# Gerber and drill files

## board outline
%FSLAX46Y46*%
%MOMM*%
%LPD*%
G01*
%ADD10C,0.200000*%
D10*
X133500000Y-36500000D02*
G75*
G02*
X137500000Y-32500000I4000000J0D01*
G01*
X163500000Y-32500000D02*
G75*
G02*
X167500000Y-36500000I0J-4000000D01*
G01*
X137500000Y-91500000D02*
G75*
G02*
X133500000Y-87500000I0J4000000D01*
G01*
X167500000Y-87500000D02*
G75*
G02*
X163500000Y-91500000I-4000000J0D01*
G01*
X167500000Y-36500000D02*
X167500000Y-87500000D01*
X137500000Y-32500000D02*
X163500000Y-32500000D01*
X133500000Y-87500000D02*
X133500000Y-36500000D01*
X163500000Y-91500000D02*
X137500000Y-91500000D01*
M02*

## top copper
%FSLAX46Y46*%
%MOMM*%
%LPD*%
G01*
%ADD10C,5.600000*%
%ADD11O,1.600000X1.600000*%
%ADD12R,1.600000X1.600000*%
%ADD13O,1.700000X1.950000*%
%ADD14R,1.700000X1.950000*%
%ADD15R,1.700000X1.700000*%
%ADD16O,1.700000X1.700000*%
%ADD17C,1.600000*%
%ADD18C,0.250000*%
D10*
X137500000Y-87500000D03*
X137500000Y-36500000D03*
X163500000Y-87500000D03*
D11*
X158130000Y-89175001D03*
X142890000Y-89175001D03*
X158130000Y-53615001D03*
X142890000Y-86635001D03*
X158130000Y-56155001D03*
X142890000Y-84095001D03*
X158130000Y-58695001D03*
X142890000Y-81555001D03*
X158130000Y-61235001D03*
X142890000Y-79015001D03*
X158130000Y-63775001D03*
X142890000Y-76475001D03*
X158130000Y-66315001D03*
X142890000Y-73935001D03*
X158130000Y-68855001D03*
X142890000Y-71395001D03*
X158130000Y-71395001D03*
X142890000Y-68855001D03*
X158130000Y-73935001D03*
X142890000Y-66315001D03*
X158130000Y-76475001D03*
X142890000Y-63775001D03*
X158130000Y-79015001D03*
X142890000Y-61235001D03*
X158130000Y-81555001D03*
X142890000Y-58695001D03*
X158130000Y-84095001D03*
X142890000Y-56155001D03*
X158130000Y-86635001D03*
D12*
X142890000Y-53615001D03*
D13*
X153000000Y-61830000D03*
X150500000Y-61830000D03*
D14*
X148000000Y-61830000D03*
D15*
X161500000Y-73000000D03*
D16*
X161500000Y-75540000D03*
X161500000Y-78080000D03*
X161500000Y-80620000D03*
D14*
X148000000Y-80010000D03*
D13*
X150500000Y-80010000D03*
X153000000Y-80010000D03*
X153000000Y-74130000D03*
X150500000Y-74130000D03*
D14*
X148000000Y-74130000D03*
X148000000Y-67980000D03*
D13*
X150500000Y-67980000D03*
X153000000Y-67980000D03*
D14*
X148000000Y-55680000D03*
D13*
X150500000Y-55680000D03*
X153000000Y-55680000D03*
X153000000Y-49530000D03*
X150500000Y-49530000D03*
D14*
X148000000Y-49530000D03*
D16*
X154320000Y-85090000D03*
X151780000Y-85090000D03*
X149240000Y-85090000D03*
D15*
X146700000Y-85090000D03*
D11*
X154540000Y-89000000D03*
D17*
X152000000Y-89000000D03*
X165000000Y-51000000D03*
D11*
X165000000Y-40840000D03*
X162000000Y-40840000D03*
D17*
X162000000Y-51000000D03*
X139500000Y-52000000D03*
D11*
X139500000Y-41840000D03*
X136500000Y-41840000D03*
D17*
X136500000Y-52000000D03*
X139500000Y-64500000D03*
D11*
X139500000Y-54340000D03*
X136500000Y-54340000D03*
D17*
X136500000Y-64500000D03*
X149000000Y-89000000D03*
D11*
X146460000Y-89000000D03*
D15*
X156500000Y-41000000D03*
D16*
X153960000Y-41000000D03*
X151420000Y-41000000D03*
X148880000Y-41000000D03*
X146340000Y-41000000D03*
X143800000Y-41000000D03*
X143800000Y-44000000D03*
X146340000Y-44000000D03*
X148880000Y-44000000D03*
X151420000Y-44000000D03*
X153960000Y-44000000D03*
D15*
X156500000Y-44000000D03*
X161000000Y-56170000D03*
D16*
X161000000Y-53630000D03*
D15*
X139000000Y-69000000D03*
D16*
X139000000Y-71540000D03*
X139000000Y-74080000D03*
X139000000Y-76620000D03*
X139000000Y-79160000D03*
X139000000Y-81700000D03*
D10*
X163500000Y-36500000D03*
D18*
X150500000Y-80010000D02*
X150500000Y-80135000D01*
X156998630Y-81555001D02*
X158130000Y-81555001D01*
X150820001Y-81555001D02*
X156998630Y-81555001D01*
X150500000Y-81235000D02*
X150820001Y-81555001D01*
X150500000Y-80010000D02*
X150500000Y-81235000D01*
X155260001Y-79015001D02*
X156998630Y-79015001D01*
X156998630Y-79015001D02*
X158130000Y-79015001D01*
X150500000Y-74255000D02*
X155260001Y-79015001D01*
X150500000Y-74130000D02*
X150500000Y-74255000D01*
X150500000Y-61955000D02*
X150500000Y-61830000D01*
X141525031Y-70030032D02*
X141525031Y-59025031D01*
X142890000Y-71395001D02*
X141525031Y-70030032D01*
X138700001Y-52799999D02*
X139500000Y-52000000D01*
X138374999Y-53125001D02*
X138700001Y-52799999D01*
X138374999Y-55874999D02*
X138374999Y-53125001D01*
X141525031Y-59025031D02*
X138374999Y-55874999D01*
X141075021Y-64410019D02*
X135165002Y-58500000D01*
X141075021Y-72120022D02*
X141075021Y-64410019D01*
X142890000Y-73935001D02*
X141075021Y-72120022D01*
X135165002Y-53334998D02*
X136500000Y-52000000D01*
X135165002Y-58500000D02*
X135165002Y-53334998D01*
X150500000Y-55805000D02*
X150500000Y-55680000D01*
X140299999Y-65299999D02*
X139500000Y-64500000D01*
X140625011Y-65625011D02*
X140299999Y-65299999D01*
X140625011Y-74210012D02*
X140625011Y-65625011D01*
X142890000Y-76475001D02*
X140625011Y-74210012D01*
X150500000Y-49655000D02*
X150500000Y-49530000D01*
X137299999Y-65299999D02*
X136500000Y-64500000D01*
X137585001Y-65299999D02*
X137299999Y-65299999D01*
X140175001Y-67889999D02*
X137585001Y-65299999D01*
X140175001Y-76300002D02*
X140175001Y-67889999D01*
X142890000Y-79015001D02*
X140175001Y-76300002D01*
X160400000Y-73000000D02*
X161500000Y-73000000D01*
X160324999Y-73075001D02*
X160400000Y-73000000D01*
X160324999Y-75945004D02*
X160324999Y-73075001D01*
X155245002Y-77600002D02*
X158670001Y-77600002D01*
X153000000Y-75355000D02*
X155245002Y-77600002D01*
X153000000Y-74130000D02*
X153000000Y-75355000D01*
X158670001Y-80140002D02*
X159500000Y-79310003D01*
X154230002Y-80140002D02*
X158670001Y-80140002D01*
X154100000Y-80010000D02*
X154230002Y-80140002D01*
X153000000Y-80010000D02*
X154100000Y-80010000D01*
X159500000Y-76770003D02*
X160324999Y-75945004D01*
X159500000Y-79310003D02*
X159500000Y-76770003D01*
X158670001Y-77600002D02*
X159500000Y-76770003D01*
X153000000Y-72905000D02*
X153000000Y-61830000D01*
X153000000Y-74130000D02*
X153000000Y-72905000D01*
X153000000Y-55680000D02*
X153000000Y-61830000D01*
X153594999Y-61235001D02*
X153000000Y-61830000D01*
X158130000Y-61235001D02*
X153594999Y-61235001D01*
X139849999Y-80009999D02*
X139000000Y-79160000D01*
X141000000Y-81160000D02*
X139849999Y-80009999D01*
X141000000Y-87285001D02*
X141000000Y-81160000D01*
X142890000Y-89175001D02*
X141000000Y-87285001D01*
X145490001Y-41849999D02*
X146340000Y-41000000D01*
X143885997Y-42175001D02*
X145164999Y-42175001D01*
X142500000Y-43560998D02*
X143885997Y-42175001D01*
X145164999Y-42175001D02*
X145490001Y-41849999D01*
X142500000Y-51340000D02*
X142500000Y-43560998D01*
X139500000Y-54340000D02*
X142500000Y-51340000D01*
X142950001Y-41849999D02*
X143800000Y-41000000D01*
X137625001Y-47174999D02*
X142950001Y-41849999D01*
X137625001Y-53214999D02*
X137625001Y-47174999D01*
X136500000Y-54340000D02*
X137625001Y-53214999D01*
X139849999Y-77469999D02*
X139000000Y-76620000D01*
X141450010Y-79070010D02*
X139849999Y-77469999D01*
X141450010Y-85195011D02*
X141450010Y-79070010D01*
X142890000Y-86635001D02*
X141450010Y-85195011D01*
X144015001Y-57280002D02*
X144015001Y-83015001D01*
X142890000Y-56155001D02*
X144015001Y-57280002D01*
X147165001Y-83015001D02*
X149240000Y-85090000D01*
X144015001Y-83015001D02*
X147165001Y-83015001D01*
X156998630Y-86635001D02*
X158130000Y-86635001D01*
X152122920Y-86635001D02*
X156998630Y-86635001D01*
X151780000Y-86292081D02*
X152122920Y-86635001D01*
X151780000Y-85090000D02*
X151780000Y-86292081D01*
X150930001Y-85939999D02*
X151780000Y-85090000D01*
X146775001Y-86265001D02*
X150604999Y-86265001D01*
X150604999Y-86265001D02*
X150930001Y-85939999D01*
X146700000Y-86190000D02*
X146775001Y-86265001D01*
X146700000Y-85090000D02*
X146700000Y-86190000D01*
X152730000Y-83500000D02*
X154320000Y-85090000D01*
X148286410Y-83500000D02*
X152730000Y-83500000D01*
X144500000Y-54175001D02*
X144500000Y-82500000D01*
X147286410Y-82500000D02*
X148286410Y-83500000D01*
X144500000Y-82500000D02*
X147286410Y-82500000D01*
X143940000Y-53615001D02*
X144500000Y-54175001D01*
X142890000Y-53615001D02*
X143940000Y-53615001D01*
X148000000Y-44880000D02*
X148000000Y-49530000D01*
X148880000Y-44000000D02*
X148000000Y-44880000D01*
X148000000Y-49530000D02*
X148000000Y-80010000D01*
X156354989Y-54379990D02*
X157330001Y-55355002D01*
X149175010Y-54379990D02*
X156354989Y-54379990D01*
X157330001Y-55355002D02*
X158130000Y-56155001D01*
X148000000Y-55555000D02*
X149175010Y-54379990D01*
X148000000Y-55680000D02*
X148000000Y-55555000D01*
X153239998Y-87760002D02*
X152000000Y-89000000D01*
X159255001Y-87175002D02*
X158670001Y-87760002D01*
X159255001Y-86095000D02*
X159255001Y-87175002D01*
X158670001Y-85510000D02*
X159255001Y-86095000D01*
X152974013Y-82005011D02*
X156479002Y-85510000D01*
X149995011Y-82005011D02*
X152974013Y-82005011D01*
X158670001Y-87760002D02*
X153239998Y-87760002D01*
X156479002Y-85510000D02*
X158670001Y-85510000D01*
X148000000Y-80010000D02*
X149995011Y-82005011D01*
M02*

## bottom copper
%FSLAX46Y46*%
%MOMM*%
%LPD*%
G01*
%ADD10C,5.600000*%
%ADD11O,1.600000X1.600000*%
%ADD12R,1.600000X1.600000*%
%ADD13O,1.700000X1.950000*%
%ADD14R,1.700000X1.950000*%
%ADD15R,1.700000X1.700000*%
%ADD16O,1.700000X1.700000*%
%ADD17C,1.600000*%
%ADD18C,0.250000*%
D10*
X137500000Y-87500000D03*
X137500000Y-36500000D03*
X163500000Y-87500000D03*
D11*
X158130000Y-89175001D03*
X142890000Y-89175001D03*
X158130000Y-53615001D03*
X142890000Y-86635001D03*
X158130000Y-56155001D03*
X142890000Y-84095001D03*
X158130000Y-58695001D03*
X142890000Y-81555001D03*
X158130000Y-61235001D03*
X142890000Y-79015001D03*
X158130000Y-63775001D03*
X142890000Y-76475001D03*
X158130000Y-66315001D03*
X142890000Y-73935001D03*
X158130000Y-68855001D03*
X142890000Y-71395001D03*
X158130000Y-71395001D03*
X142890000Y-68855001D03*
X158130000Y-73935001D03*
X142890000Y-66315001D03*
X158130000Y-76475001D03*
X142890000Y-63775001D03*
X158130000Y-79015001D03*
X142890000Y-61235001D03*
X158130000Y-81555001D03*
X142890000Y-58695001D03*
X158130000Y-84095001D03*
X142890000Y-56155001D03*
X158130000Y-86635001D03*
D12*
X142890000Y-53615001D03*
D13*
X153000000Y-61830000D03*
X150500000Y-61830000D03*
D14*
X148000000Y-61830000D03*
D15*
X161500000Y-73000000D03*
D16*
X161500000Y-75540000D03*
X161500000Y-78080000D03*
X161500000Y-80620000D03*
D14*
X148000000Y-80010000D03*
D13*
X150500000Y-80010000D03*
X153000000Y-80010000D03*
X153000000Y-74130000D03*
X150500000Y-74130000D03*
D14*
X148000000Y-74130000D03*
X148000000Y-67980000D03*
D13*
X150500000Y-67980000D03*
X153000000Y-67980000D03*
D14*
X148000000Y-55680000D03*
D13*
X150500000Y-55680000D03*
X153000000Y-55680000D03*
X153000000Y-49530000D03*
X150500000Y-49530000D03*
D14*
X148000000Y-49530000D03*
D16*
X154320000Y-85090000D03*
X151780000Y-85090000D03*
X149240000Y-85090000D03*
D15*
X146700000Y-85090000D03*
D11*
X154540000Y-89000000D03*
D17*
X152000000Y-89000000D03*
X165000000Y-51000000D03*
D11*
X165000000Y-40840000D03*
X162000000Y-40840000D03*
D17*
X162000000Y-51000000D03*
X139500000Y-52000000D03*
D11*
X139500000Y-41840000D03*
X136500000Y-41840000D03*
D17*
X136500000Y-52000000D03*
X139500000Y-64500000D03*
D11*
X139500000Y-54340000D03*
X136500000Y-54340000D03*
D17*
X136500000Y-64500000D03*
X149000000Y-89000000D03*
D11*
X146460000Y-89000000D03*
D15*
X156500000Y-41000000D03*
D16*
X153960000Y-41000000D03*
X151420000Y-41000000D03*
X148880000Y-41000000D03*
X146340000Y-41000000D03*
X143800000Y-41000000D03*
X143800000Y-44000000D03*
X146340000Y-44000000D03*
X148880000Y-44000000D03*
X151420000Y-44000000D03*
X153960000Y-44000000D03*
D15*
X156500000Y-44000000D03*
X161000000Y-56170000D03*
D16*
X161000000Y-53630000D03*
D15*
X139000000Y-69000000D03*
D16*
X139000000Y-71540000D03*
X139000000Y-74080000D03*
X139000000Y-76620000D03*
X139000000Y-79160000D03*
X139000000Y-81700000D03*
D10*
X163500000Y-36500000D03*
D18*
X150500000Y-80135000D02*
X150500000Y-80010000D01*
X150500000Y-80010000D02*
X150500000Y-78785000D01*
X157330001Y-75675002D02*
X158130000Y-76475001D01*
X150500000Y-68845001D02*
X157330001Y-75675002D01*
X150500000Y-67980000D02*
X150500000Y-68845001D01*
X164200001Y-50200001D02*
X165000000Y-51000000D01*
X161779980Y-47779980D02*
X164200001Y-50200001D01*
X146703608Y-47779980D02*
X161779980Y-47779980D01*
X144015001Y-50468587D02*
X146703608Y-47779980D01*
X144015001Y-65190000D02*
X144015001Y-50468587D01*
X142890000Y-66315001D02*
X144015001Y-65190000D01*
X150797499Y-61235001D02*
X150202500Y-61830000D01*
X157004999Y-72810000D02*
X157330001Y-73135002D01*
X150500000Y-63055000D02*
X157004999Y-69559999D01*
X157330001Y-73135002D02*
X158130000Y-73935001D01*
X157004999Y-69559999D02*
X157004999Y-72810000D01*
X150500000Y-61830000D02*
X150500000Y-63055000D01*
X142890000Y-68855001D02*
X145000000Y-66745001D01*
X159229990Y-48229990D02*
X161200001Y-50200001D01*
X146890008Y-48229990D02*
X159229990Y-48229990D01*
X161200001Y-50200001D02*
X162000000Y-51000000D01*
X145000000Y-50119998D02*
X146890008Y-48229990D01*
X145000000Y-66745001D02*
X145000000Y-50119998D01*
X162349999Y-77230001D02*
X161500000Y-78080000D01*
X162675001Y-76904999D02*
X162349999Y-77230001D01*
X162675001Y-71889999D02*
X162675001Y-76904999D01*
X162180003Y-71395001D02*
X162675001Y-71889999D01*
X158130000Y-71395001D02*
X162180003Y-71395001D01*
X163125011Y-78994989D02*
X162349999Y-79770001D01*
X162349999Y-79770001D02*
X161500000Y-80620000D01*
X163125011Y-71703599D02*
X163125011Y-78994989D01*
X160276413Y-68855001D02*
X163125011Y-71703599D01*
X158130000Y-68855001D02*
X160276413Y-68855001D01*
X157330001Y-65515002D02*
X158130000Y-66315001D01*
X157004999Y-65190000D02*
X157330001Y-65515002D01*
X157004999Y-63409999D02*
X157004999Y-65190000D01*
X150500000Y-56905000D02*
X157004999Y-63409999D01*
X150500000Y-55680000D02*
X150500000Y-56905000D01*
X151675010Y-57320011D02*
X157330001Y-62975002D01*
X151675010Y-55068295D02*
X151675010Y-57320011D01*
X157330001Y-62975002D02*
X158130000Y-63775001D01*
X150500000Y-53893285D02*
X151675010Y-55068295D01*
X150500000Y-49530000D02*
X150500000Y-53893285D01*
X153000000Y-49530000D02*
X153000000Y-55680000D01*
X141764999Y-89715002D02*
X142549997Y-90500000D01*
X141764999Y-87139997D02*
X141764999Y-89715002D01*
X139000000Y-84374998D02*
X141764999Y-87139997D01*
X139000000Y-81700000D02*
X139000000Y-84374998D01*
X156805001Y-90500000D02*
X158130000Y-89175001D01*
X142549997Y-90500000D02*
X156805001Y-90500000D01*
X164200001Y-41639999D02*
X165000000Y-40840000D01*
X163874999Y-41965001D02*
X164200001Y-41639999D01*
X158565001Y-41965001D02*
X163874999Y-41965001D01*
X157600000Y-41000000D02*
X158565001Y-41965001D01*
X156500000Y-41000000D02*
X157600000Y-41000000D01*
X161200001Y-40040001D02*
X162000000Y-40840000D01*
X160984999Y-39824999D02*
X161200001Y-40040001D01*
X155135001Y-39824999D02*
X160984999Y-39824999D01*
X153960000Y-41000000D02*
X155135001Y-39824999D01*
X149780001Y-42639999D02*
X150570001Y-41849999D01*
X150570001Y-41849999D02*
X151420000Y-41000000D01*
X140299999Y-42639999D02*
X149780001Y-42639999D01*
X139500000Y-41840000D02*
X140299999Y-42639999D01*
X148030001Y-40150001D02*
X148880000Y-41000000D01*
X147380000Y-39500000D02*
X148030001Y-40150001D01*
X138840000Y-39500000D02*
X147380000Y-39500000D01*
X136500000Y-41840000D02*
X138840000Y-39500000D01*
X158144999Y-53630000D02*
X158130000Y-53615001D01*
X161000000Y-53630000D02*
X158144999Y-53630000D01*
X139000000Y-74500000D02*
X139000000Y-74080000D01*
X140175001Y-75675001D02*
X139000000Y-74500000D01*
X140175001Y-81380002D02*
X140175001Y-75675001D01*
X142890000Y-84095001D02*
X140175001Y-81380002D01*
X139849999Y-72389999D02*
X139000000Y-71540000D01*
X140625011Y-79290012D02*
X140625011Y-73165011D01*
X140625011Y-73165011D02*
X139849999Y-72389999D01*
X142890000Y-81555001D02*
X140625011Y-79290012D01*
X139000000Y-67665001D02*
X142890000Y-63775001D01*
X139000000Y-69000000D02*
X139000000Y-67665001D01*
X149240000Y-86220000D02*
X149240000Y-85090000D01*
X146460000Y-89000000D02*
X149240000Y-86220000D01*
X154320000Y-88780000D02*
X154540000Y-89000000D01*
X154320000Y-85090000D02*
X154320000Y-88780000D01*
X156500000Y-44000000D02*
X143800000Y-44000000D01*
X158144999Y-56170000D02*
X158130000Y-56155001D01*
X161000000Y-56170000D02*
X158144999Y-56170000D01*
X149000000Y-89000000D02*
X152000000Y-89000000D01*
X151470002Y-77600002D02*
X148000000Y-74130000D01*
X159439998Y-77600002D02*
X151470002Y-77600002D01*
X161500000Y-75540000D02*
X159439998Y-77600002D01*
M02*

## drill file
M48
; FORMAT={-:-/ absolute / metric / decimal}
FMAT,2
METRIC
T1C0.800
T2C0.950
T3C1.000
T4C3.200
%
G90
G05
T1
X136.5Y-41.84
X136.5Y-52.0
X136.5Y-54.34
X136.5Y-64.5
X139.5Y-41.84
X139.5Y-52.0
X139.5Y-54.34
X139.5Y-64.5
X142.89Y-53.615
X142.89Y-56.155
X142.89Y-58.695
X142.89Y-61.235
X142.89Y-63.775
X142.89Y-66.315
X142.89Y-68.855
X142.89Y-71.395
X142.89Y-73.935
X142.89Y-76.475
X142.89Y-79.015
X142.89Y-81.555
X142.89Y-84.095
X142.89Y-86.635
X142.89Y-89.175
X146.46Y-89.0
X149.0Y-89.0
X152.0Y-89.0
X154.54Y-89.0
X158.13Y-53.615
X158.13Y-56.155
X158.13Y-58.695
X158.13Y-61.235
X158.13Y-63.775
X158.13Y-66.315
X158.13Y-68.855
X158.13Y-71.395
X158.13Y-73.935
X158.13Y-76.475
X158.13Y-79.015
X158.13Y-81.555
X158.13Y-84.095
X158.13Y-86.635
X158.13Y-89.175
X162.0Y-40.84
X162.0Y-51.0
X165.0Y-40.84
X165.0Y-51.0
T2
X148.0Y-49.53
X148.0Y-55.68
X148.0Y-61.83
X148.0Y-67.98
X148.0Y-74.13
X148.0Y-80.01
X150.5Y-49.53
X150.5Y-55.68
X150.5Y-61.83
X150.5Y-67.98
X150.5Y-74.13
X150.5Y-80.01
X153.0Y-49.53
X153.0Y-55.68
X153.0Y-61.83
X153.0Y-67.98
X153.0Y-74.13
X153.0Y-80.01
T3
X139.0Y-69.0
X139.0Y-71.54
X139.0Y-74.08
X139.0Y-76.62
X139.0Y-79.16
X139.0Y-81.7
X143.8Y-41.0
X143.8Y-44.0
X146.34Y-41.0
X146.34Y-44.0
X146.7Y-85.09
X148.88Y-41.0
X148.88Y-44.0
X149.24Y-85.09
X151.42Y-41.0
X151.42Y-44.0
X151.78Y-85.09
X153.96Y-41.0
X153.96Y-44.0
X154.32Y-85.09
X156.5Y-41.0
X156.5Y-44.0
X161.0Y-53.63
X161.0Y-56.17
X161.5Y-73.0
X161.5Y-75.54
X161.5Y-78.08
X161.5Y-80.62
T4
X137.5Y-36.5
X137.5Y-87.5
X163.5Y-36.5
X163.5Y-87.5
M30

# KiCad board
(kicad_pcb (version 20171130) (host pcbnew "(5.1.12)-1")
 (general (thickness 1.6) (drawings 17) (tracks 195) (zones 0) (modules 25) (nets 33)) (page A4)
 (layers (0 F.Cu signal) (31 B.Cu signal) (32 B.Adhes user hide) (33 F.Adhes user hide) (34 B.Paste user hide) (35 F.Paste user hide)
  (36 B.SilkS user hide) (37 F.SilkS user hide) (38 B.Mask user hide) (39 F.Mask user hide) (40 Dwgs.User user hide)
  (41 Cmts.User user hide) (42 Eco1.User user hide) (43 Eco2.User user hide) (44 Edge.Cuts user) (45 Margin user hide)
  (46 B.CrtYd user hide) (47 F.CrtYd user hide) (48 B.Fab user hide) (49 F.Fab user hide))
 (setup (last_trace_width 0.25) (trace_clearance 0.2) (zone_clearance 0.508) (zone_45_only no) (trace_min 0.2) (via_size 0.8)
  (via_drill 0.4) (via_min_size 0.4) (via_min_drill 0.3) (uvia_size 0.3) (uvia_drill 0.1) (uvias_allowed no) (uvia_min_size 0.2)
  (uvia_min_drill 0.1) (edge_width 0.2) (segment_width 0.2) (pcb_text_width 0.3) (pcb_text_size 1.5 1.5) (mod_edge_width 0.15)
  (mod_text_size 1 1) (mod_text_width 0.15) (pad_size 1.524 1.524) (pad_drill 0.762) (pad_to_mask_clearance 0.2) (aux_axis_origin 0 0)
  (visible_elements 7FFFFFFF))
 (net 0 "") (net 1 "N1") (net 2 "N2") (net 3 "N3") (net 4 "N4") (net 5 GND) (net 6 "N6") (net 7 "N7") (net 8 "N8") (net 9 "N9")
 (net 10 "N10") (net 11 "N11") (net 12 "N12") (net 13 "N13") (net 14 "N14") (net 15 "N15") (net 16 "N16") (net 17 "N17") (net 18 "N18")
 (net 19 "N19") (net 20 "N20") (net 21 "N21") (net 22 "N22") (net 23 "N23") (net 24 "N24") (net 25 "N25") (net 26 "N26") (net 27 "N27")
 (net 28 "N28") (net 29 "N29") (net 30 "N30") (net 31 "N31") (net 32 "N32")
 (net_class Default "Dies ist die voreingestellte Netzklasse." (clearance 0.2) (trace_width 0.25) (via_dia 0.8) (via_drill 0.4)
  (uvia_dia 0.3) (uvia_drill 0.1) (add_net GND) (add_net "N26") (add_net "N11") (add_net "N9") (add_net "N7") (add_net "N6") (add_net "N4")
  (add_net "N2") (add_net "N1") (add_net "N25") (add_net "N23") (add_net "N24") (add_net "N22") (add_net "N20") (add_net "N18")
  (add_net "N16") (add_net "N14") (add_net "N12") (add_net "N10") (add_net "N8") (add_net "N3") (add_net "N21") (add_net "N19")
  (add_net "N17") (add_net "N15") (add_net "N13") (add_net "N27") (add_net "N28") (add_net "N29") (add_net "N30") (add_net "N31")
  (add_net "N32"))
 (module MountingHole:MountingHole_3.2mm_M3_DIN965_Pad (layer F.Cu) (at 137.5 87.5)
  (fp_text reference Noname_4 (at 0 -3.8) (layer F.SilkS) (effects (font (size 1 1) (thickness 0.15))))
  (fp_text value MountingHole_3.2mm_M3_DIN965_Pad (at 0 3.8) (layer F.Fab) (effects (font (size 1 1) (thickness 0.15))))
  (pad 1 thru_hole circle (at 0 0) (size 5.6 5.6) (drill 3.2) (layers *.Cu *.Mask)))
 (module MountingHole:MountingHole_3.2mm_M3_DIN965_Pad (layer F.Cu) (at 137.5 36.5)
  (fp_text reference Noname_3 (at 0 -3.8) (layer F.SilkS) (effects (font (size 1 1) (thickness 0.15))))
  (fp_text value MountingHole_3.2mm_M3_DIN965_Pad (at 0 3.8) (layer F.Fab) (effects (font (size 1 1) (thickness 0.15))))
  (pad 1 thru_hole circle (at 0 0) (size 5.6 5.6) (drill 3.2) (layers *.Cu *.Mask)))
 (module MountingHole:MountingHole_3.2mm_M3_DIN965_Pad (layer F.Cu) (at 163.5 87.5)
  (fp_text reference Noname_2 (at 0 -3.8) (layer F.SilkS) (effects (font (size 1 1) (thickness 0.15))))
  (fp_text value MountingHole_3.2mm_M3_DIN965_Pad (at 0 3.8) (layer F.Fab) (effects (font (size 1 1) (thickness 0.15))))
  (pad 1 thru_hole circle (at 0 0) (size 5.6 5.6) (drill 3.2) (layers *.Cu *.Mask)))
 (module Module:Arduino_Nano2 (layer F.Cu) (at 142.89 53.615001)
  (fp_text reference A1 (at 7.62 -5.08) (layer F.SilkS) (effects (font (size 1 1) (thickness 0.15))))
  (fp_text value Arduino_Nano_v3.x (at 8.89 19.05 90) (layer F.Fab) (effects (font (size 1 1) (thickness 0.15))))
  (pad 16 thru_hole oval (at 15.24 35.56) (size 1.6 1.6) (drill 0.8) (layers *.Cu *.Mask) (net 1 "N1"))
  (pad 15 thru_hole oval (at 0 35.56) (size 1.6 1.6) (drill 0.8) (layers *.Cu *.Mask) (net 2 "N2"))
  (pad 30 thru_hole oval (at 15.24 0) (size 1.6 1.6) (drill 0.8) (layers *.Cu *.Mask) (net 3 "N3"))
  (pad 14 thru_hole oval (at 0 33.02) (size 1.6 1.6) (drill 0.8) (layers *.Cu *.Mask) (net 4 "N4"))
  (pad 29 thru_hole oval (at 15.24 2.54) (size 1.6 1.6) (drill 0.8) (layers *.Cu *.Mask) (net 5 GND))
  (pad 13 thru_hole oval (at 0 30.48) (size 1.6 1.6) (drill 0.8) (layers *.Cu *.Mask) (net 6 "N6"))
  (pad 28 thru_hole oval (at 15.24 5.08) (size 1.6 1.6) (drill 0.8) (layers *.Cu *.Mask))
  (pad 12 thru_hole oval (at 0 27.94) (size 1.6 1.6) (drill 0.8) (layers *.Cu *.Mask) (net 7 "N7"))
  (pad 27 thru_hole oval (at 15.24 7.62) (size 1.6 1.6) (drill 0.8) (layers *.Cu *.Mask) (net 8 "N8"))
  (pad 11 thru_hole oval (at 0 25.4) (size 1.6 1.6) (drill 0.8) (layers *.Cu *.Mask) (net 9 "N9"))
  (pad 26 thru_hole oval (at 15.24 10.16) (size 1.6 1.6) (drill 0.8) (layers *.Cu *.Mask) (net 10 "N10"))
  (pad 10 thru_hole oval (at 0 22.86) (size 1.6 1.6) (drill 0.8) (layers *.Cu *.Mask) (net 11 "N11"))
  (pad 25 thru_hole oval (at 15.24 12.7) (size 1.6 1.6) (drill 0.8) (layers *.Cu *.Mask) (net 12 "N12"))
  (pad 9 thru_hole oval (at 0 20.32) (size 1.6 1.6) (drill 0.8) (layers *.Cu *.Mask) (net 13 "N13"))
  (pad 24 thru_hole oval (at 15.24 15.24) (size 1.6 1.6) (drill 0.8) (layers *.Cu *.Mask) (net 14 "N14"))
  (pad 8 thru_hole oval (at 0 17.78) (size 1.6 1.6) (drill 0.8) (layers *.Cu *.Mask) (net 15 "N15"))
  (pad 23 thru_hole oval (at 15.24 17.78) (size 1.6 1.6) (drill 0.8) (layers *.Cu *.Mask) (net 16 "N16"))
  (pad 7 thru_hole oval (at 0 15.24) (size 1.6 1.6) (drill 0.8) (layers *.Cu *.Mask) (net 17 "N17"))
  (pad 22 thru_hole oval (at 15.24 20.32) (size 1.6 1.6) (drill 0.8) (layers *.Cu *.Mask) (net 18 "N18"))
  (pad 6 thru_hole oval (at 0 12.7) (size 1.6 1.6) (drill 0.8) (layers *.Cu *.Mask) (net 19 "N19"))
  (pad 21 thru_hole oval (at 15.24 22.86) (size 1.6 1.6) (drill 0.8) (layers *.Cu *.Mask) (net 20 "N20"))
  (pad 5 thru_hole oval (at 0 10.16) (size 1.6 1.6) (drill 0.8) (layers *.Cu *.Mask) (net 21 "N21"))
  (pad 20 thru_hole oval (at 15.24 25.4) (size 1.6 1.6) (drill 0.8) (layers *.Cu *.Mask) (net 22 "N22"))
  (pad 4 thru_hole oval (at 0 7.62) (size 1.6 1.6) (drill 0.8) (layers *.Cu *.Mask))
  (pad 19 thru_hole oval (at 15.24 27.94) (size 1.6 1.6) (drill 0.8) (layers *.Cu *.Mask) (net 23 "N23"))
  (pad 3 thru_hole oval (at 0 5.08) (size 1.6 1.6) (drill 0.8) (layers *.Cu *.Mask))
  (pad 18 thru_hole oval (at 15.24 30.48) (size 1.6 1.6) (drill 0.8) (layers *.Cu *.Mask))
  (pad 2 thru_hole oval (at 0 2.54) (size 1.6 1.6) (drill 0.8) (layers *.Cu *.Mask) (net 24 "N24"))
  (pad 17 thru_hole oval (at 15.24 33.02) (size 1.6 1.6) (drill 0.8) (layers *.Cu *.Mask) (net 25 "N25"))
  (pad 1 thru_hole rect (at 0 0) (size 1.6 1.6) (drill 0.8) (layers *.Cu *.Mask) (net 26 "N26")))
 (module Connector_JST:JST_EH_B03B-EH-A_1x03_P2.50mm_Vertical (layer F.Cu) (at 148 61.83)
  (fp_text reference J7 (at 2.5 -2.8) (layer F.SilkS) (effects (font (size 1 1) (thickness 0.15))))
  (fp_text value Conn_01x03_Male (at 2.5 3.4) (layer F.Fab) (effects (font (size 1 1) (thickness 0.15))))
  (pad 3 thru_hole oval (at 5 0) (size 1.7 1.95) (drill 0.95) (layers *.Cu *.Mask) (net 8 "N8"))
  (pad 2 thru_hole oval (at 2.5 0) (size 1.7 1.95) (drill 0.95) (layers *.Cu *.Mask) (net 18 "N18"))
  (pad 1 thru_hole rect (at 0 0) (size 1.7 1.95) (drill 0.95) (layers *.Cu *.Mask) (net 5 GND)))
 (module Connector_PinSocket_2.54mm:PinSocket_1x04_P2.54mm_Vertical (layer F.Cu) (at 161.5 73)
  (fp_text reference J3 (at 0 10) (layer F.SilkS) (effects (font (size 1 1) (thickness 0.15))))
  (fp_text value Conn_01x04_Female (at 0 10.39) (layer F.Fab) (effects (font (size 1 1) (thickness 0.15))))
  (pad 1 thru_hole rect (at 0 0) (size 1.7 1.7) (drill 1) (layers *.Cu *.Mask) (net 8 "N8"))
  (pad 2 thru_hole oval (at 0 2.54) (size 1.7 1.7) (drill 1) (layers *.Cu *.Mask) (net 5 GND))
  (pad 3 thru_hole oval (at 0 5.08) (size 1.7 1.7) (drill 1) (layers *.Cu *.Mask) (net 16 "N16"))
  (pad 4 thru_hole oval (at 0 7.62) (size 1.7 1.7) (drill 1) (layers *.Cu *.Mask) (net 14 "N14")))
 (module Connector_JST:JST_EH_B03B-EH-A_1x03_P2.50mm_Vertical (layer F.Cu) (at 148 80.01)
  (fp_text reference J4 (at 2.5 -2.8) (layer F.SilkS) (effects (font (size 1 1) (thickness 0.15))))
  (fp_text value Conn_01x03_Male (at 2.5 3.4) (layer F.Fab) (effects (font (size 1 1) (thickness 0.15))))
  (pad 1 thru_hole rect (at 0 0) (size 1.7 1.95) (drill 0.95) (layers *.Cu *.Mask) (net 5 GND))
  (pad 2 thru_hole oval (at 2.5 0) (size 1.7 1.95) (drill 0.95) (layers *.Cu *.Mask) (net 23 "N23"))
  (pad 3 thru_hole oval (at 5 0) (size 1.7 1.95) (drill 0.95) (layers *.Cu *.Mask) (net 8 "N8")))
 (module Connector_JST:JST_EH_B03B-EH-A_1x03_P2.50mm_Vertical (layer F.Cu) (at 148 74.13)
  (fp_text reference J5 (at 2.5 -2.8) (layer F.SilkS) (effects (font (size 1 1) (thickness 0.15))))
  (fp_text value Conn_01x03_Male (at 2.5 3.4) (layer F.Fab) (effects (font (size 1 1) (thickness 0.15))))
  (pad 3 thru_hole oval (at 5 0) (size 1.7 1.95) (drill 0.95) (layers *.Cu *.Mask) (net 8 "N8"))
  (pad 2 thru_hole oval (at 2.5 0) (size 1.7 1.95) (drill 0.95) (layers *.Cu *.Mask) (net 22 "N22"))
  (pad 1 thru_hole rect (at 0 0) (size 1.7 1.95) (drill 0.95) (layers *.Cu *.Mask) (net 5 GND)))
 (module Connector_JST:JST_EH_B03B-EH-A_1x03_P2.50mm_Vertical (layer F.Cu) (at 148 67.98)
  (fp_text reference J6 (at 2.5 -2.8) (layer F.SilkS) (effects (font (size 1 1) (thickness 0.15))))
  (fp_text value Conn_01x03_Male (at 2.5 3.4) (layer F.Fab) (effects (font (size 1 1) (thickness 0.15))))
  (pad 1 thru_hole rect (at 0 0) (size 1.7 1.95) (drill 0.95) (layers *.Cu *.Mask) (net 5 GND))
  (pad 2 thru_hole oval (at 2.5 0) (size 1.7 1.95) (drill 0.95) (layers *.Cu *.Mask) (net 20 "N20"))
  (pad 3 thru_hole oval (at 5 0) (size 1.7 1.95) (drill 0.95) (layers *.Cu *.Mask) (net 8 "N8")))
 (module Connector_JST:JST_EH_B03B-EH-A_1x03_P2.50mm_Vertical (layer F.Cu) (at 148 55.68)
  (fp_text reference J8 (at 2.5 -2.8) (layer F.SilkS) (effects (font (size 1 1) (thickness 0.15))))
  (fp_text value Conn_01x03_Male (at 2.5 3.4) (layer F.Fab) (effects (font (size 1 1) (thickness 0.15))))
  (pad 1 thru_hole rect (at 0 0) (size 1.7 1.95) (drill 0.95) (layers *.Cu *.Mask) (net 5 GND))
  (pad 2 thru_hole oval (at 2.5 0) (size 1.7 1.95) (drill 0.95) (layers *.Cu *.Mask) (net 12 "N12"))
  (pad 3 thru_hole oval (at 5 0) (size 1.7 1.95) (drill 0.95) (layers *.Cu *.Mask) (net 8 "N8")))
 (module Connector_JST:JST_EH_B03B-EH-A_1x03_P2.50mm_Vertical (layer F.Cu) (at 148 49.53)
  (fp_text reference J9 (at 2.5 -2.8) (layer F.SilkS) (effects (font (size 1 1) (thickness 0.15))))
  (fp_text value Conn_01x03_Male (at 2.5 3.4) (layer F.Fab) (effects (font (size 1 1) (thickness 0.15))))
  (pad 3 thru_hole oval (at 5 0) (size 1.7 1.95) (drill 0.95) (layers *.Cu *.Mask) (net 8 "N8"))
  (pad 2 thru_hole oval (at 2.5 0) (size 1.7 1.95) (drill 0.95) (layers *.Cu *.Mask) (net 10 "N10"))
  (pad 1 thru_hole rect (at 0 0) (size 1.7 1.95) (drill 0.95) (layers *.Cu *.Mask) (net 5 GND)))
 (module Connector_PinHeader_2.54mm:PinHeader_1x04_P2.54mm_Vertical (layer F.Cu) (at 146.7 85.09 90)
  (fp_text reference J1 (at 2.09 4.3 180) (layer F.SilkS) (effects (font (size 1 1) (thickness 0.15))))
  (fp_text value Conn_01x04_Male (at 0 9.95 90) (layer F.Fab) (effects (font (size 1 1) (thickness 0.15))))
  (pad 4 thru_hole oval (at 0 7.62 90) (size 1.7 1.7) (drill 1) (layers *.Cu *.Mask) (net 26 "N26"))
  (pad 3 thru_hole oval (at 0 5.08 90) (size 1.7 1.7) (drill 1) (layers *.Cu *.Mask) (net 25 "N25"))
  (pad 2 thru_hole oval (at 0 2.54 90) (size 1.7 1.7) (drill 1) (layers *.Cu *.Mask) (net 24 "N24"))
  (pad 1 thru_hole rect (at 0 0 90) (size 1.7 1.7) (drill 1) (layers *.Cu *.Mask) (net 25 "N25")))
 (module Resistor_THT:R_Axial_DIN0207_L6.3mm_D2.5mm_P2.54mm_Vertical (layer F.Cu) (at 152 89)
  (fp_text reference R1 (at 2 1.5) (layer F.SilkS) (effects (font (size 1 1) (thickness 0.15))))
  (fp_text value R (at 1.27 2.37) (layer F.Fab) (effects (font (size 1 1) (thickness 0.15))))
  (pad 2 thru_hole oval (at 2.54 0) (size 1.6 1.6) (drill 0.8) (layers *.Cu *.Mask) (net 26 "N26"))
  (pad 1 thru_hole circle (at 0 0) (size 1.6 1.6) (drill 0.8) (layers *.Cu *.Mask) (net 5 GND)))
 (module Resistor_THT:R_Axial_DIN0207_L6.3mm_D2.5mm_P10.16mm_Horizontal (layer F.Cu) (at 165 51 90)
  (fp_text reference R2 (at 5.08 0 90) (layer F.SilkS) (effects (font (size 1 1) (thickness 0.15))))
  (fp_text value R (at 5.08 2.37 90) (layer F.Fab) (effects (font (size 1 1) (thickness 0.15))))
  (pad 1 thru_hole circle (at 0 0 90) (size 1.6 1.6) (drill 0.8) (layers *.Cu *.Mask) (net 19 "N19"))
  (pad 2 thru_hole oval (at 10.16 0 90) (size 1.6 1.6) (drill 0.8) (layers *.Cu *.Mask) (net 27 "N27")))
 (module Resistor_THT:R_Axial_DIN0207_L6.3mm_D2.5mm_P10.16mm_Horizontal (layer F.Cu) (at 162 51 90)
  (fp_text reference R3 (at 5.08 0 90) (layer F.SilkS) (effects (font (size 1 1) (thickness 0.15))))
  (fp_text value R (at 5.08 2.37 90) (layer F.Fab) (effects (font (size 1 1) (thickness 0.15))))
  (pad 2 thru_hole oval (at 10.16 0 90) (size 1.6 1.6) (drill 0.8) (layers *.Cu *.Mask) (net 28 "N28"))
  (pad 1 thru_hole circle (at 0 0 90) (size 1.6 1.6) (drill 0.8) (layers *.Cu *.Mask) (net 17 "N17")))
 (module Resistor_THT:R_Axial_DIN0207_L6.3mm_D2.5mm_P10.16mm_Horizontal (layer F.Cu) (at 139.5 52 90)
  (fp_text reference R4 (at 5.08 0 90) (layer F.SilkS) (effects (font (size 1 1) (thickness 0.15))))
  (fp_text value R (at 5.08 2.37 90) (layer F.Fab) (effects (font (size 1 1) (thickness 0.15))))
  (pad 1 thru_hole circle (at 0 0 90) (size 1.6 1.6) (drill 0.8) (layers *.Cu *.Mask) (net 15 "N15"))
  (pad 2 thru_hole oval (at 10.16 0 90) (size 1.6 1.6) (drill 0.8) (layers *.Cu *.Mask) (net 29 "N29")))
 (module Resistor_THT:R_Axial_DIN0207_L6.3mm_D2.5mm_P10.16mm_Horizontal (layer F.Cu) (at 136.5 52 90)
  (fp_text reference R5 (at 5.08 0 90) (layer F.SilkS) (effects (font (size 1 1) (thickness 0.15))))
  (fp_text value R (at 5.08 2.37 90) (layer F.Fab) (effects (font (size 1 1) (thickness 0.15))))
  (pad 2 thru_hole oval (at 10.16 0 90) (size 1.6 1.6) (drill 0.8) (layers *.Cu *.Mask) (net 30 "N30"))
  (pad 1 thru_hole circle (at 0 0 90) (size 1.6 1.6) (drill 0.8) (layers *.Cu *.Mask) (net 13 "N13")))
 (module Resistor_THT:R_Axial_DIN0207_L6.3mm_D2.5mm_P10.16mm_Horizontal (layer F.Cu) (at 139.5 64.5 90)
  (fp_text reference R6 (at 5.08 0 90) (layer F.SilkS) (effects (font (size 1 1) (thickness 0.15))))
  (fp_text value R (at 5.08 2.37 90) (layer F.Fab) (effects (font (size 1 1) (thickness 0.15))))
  (pad 1 thru_hole circle (at 0 0 90) (size 1.6 1.6) (drill 0.8) (layers *.Cu *.Mask) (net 11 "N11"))
  (pad 2 thru_hole oval (at 10.16 0 90) (size 1.6 1.6) (drill 0.8) (layers *.Cu *.Mask) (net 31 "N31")))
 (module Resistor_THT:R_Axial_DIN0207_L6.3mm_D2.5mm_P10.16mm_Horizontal (layer F.Cu) (at 136.5 64.5 90)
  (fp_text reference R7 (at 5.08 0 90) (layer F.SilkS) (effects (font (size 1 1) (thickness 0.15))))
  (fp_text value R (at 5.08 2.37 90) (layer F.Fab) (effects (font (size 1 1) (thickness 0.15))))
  (pad 2 thru_hole oval (at 10.16 0 90) (size 1.6 1.6) (drill 0.8) (layers *.Cu *.Mask) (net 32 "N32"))
  (pad 1 thru_hole circle (at 0 0 90) (size 1.6 1.6) (drill 0.8) (layers *.Cu *.Mask) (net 9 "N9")))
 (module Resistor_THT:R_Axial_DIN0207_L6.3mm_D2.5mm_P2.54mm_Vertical (layer F.Cu) (at 149 89 180)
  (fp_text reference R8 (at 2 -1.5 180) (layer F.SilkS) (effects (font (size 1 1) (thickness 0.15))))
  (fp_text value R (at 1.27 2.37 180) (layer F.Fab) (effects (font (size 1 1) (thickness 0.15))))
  (pad 1 thru_hole circle (at 0 0 180) (size 1.6 1.6) (drill 0.8) (layers *.Cu *.Mask) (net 5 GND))
  (pad 2 thru_hole oval (at 2.54 0 180) (size 1.6 1.6) (drill 0.8) (layers *.Cu *.Mask) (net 24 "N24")))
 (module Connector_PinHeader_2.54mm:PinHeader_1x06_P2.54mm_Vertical (layer F.Cu) (at 156.5 41 270)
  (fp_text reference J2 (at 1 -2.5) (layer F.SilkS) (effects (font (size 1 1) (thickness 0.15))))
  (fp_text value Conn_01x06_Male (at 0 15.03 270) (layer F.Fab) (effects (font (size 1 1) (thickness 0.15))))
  (pad 1 thru_hole rect (at 0 0 270) (size 1.7 1.7) (drill 1) (layers *.Cu *.Mask) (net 27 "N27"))
  (pad 2 thru_hole oval (at 0 2.54 270) (size 1.7 1.7) (drill 1) (layers *.Cu *.Mask) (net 28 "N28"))
  (pad 3 thru_hole oval (at 0 5.08 270) (size 1.7 1.7) (drill 1) (layers *.Cu *.Mask) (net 29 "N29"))
  (pad 4 thru_hole oval (at 0 7.62 270) (size 1.7 1.7) (drill 1) (layers *.Cu *.Mask) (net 30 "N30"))
  (pad 5 thru_hole oval (at 0 10.16 270) (size 1.7 1.7) (drill 1) (layers *.Cu *.Mask) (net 31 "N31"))
  (pad 6 thru_hole oval (at 0 12.7 270) (size 1.7 1.7) (drill 1) (layers *.Cu *.Mask) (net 32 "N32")))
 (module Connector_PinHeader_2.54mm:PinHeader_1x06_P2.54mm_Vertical (layer F.Cu) (at 156.5 44 270)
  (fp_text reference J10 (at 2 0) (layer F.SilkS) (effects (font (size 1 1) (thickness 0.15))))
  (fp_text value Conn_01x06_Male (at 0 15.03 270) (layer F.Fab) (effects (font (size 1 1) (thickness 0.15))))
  (pad 6 thru_hole oval (at 0 12.7 270) (size 1.7 1.7) (drill 1) (layers *.Cu *.Mask) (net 5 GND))
  (pad 5 thru_hole oval (at 0 10.16 270) (size 1.7 1.7) (drill 1) (layers *.Cu *.Mask) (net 5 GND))
  (pad 4 thru_hole oval (at 0 7.62 270) (size 1.7 1.7) (drill 1) (layers *.Cu *.Mask) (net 5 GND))
  (pad 3 thru_hole oval (at 0 5.08 270) (size 1.7 1.7) (drill 1) (layers *.Cu *.Mask) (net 5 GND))
  (pad 2 thru_hole oval (at 0 2.54 270) (size 1.7 1.7) (drill 1) (layers *.Cu *.Mask) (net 5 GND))
  (pad 1 thru_hole rect (at 0 0 270) (size 1.7 1.7) (drill 1) (layers *.Cu *.Mask) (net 5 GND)))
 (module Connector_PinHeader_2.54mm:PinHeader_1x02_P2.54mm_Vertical (layer F.Cu) (at 161 56.17 180)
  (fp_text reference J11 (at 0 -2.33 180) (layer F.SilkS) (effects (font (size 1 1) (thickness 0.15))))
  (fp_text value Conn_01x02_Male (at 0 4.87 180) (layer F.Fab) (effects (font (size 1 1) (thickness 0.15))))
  (pad 1 thru_hole rect (at 0 0 180) (size 1.7 1.7) (drill 1) (layers *.Cu *.Mask) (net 5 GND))
  (pad 2 thru_hole oval (at 0 2.54 180) (size 1.7 1.7) (drill 1) (layers *.Cu *.Mask) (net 3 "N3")))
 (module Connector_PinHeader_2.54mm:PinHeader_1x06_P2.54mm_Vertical (layer F.Cu) (at 139 69)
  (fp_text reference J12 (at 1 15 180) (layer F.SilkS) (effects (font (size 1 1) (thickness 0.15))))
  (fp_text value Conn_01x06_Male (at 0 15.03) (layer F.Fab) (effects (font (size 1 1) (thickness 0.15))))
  (pad 1 thru_hole rect (at 0 0) (size 1.7 1.7) (drill 1) (layers *.Cu *.Mask) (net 21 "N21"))
  (pad 2 thru_hole oval (at 0 2.54) (size 1.7 1.7) (drill 1) (layers *.Cu *.Mask) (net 7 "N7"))
  (pad 3 thru_hole oval (at 0 5.08) (size 1.7 1.7) (drill 1) (layers *.Cu *.Mask) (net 6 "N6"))
  (pad 4 thru_hole oval (at 0 7.62) (size 1.7 1.7) (drill 1) (layers *.Cu *.Mask) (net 4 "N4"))
  (pad 5 thru_hole oval (at 0 10.16) (size 1.7 1.7) (drill 1) (layers *.Cu *.Mask) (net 2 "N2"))
  (pad 6 thru_hole oval (at 0 12.7) (size 1.7 1.7) (drill 1) (layers *.Cu *.Mask) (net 1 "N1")))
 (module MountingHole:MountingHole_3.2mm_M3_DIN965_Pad (layer F.Cu) (at 163.5 36.5)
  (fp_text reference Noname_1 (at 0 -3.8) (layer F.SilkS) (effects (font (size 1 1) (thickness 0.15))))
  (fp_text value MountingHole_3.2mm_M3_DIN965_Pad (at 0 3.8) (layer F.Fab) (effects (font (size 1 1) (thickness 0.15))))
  (pad 1 thru_hole circle (at 0 0) (size 5.6 5.6) (drill 3.2) (layers *.Cu *.Mask)))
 (gr_arc (start 137.5 36.5) (end 137.5 32.5) (angle -90) (layer Edge.Cuts) (width 0.2))
 (gr_arc (start 163.5 36.5) (end 167.5 36.5) (angle -90) (layer Edge.Cuts) (width 0.2))
 (gr_arc (start 137.5 87.5) (end 133.5 87.5) (angle -90) (layer Edge.Cuts) (width 0.2))
 (gr_arc (start 163.5 87.5) (end 163.5 91.5) (angle -90) (layer Edge.Cuts) (width 0.2))
 (gr_line (start 167.5 36.5) (end 167.5 87.5) (layer Edge.Cuts) (width 0.2))
 (gr_line (start 137.5 32.5) (end 163.5 32.5) (layer Edge.Cuts) (width 0.2))
 (gr_line (start 133.5 87.5) (end 133.5 36.5) (layer Edge.Cuts) (width 0.2))
 (gr_line (start 163.5 91.5) (end 137.5 91.5) (layer Edge.Cuts) (width 0.2))
 (segment (start 150.5 80.01) (end 150.5 80.135) (width 0.25) (layer F.Cu) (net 23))
 (segment (start 150.5 80.135) (end 150.5 80.01) (width 0.25) (layer B.Cu) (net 23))
 (segment (start 150.5 80.01) (end 150.5 78.785) (width 0.25) (layer B.Cu) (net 23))
 (segment (start 156.99863 81.555001) (end 158.13 81.555001) (width 0.25) (layer F.Cu) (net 23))
 (segment (start 150.820001 81.555001) (end 156.99863 81.555001) (width 0.25) (layer F.Cu) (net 23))
 (segment (start 150.5 81.235) (end 150.820001 81.555001) (width 0.25) (layer F.Cu) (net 23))
 (segment (start 150.5 80.01) (end 150.5 81.235) (width 0.25) (layer F.Cu) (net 23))
 (segment (start 155.260001 79.015001) (end 156.99863 79.015001) (width 0.25) (layer F.Cu) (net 22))
 (segment (start 156.99863 79.015001) (end 158.13 79.015001) (width 0.25) (layer F.Cu) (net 22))
 (segment (start 150.5 74.255) (end 155.260001 79.015001) (width 0.25) (layer F.Cu) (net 22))
 (segment (start 150.5 74.13) (end 150.5 74.255) (width 0.25) (layer F.Cu) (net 22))
 (segment (start 157.330001 75.675002) (end 158.13 76.475001) (width 0.25) (layer B.Cu) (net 20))
 (segment (start 150.5 68.845001) (end 157.330001 75.675002) (width 0.25) (layer B.Cu) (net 20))
 (segment (start 150.5 67.98) (end 150.5 68.845001) (width 0.25) (layer B.Cu) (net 20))
 (segment (start 164.200001 50.200001) (end 165 51) (width 0.25) (layer B.Cu) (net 19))
 (segment (start 161.77998 47.77998) (end 164.200001 50.200001) (width 0.25) (layer B.Cu) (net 19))
 (segment (start 146.703608 47.77998) (end 161.77998 47.77998) (width 0.25) (layer B.Cu) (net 19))
 (segment (start 144.015001 50.468587) (end 146.703608 47.77998) (width 0.25) (layer B.Cu) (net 19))
 (segment (start 144.015001 65.19) (end 144.015001 50.468587) (width 0.25) (layer B.Cu) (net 19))
 (segment (start 142.89 66.315001) (end 144.015001 65.19) (width 0.25) (layer B.Cu) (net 19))
 (segment (start 150.5 61.955) (end 150.5 61.83) (width 0.25) (layer F.Cu) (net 18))
 (segment (start 150.797499 61.235001) (end 150.2025 61.83) (width 0.25) (layer B.Cu) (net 18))
 (segment (start 157.004999 72.81) (end 157.330001 73.135002) (width 0.25) (layer B.Cu) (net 18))
 (segment (start 150.5 63.055) (end 157.004999 69.559999) (width 0.25) (layer B.Cu) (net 18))
 (segment (start 157.330001 73.135002) (end 158.13 73.935001) (width 0.25) (layer B.Cu) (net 18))
 (segment (start 157.004999 69.559999) (end 157.004999 72.81) (width 0.25) (layer B.Cu) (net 18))
 (segment (start 150.5 61.83) (end 150.5 63.055) (width 0.25) (layer B.Cu) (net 18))
 (segment (start 142.89 68.855001) (end 145 66.745001) (width 0.25) (layer B.Cu) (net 17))
 (segment (start 159.22999 48.22999) (end 161.200001 50.200001) (width 0.25) (layer B.Cu) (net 17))
 (segment (start 146.890008 48.22999) (end 159.22999 48.22999) (width 0.25) (layer B.Cu) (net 17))
 (segment (start 161.200001 50.200001) (end 162 51) (width 0.25) (layer B.Cu) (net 17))
 (segment (start 145 50.119998) (end 146.890008 48.22999) (width 0.25) (layer B.Cu) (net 17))
 (segment (start 145 66.745001) (end 145 50.119998) (width 0.25) (layer B.Cu) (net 17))
 (segment (start 162.349999 77.230001) (end 161.5 78.08) (width 0.25) (layer B.Cu) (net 16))
 (segment (start 162.675001 76.904999) (end 162.349999 77.230001) (width 0.25) (layer B.Cu) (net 16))
 (segment (start 162.675001 71.889999) (end 162.675001 76.904999) (width 0.25) (layer B.Cu) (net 16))
 (segment (start 162.180003 71.395001) (end 162.675001 71.889999) (width 0.25) (layer B.Cu) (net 16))
 (segment (start 158.13 71.395001) (end 162.180003 71.395001) (width 0.25) (layer B.Cu) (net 16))
 (segment (start 141.525031 70.030032) (end 141.525031 59.025031) (width 0.25) (layer F.Cu) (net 15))
 (segment (start 142.89 71.395001) (end 141.525031 70.030032) (width 0.25) (layer F.Cu) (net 15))
 (segment (start 138.700001 52.799999) (end 139.5 52) (width 0.25) (layer F.Cu) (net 15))
 (segment (start 138.374999 53.125001) (end 138.700001 52.799999) (width 0.25) (layer F.Cu) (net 15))
 (segment (start 138.374999 55.874999) (end 138.374999 53.125001) (width 0.25) (layer F.Cu) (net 15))
 (segment (start 141.525031 59.025031) (end 138.374999 55.874999) (width 0.25) (layer F.Cu) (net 15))
 (segment (start 163.125011 78.994989) (end 162.349999 79.770001) (width 0.25) (layer B.Cu) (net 14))
 (segment (start 162.349999 79.770001) (end 161.5 80.62) (width 0.25) (layer B.Cu) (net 14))
 (segment (start 163.125011 71.703599) (end 163.125011 78.994989) (width 0.25) (layer B.Cu) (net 14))
 (segment (start 160.276413 68.855001) (end 163.125011 71.703599) (width 0.25) (layer B.Cu) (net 14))
 (segment (start 158.13 68.855001) (end 160.276413 68.855001) (width 0.25) (layer B.Cu) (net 14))
 (segment (start 141.075021 64.410019) (end 135.165002 58.5) (width 0.25) (layer F.Cu) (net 13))
 (segment (start 141.075021 72.120022) (end 141.075021 64.410019) (width 0.25) (layer F.Cu) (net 13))
 (segment (start 142.89 73.935001) (end 141.075021 72.120022) (width 0.25) (layer F.Cu) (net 13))
 (segment (start 135.165002 53.334998) (end 136.5 52) (width 0.25) (layer F.Cu) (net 13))
 (segment (start 135.165002 58.5) (end 135.165002 53.334998) (width 0.25) (layer F.Cu) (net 13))
 (segment (start 150.5 55.805) (end 150.5 55.68) (width 0.25) (layer F.Cu) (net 12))
 (segment (start 157.330001 65.515002) (end 158.13 66.315001) (width 0.25) (layer B.Cu) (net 12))
 (segment (start 157.004999 65.19) (end 157.330001 65.515002) (width 0.25) (layer B.Cu) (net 12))
 (segment (start 157.004999 63.409999) (end 157.004999 65.19) (width 0.25) (layer B.Cu) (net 12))
 (segment (start 150.5 56.905) (end 157.004999 63.409999) (width 0.25) (layer B.Cu) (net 12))
 (segment (start 150.5 55.68) (end 150.5 56.905) (width 0.25) (layer B.Cu) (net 12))
 (segment (start 140.299999 65.299999) (end 139.5 64.5) (width 0.25) (layer F.Cu) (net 11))
 (segment (start 140.625011 65.625011) (end 140.299999 65.299999) (width 0.25) (layer F.Cu) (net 11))
 (segment (start 140.625011 74.210012) (end 140.625011 65.625011) (width 0.25) (layer F.Cu) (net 11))
 (segment (start 142.89 76.475001) (end 140.625011 74.210012) (width 0.25) (layer F.Cu) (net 11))
 (segment (start 150.5 49.655) (end 150.5 49.53) (width 0.25) (layer F.Cu) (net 10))
 (segment (start 151.67501 57.320011) (end 157.330001 62.975002) (width 0.25) (layer B.Cu) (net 10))
 (segment (start 151.67501 55.068295) (end 151.67501 57.320011) (width 0.25) (layer B.Cu) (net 10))
 (segment (start 157.330001 62.975002) (end 158.13 63.775001) (width 0.25) (layer B.Cu) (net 10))
 (segment (start 150.5 53.893285) (end 151.67501 55.068295) (width 0.25) (layer B.Cu) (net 10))
 (segment (start 150.5 49.53) (end 150.5 53.893285) (width 0.25) (layer B.Cu) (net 10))
 (segment (start 137.299999 65.299999) (end 136.5 64.5) (width 0.25) (layer F.Cu) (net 9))
 (segment (start 137.585001 65.299999) (end 137.299999 65.299999) (width 0.25) (layer F.Cu) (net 9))
 (segment (start 140.175001 67.889999) (end 137.585001 65.299999) (width 0.25) (layer F.Cu) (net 9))
 (segment (start 140.175001 76.300002) (end 140.175001 67.889999) (width 0.25) (layer F.Cu) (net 9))
 (segment (start 142.89 79.015001) (end 140.175001 76.300002) (width 0.25) (layer F.Cu) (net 9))
 (segment (start 160.4 73) (end 161.5 73) (width 0.25) (layer F.Cu) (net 8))
 (segment (start 160.324999 73.075001) (end 160.4 73) (width 0.25) (layer F.Cu) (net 8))
 (segment (start 160.324999 75.945004) (end 160.324999 73.075001) (width 0.25) (layer F.Cu) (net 8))
 (segment (start 155.245002 77.600002) (end 158.670001 77.600002) (width 0.25) (layer F.Cu) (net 8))
 (segment (start 153 75.355) (end 155.245002 77.600002) (width 0.25) (layer F.Cu) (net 8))
 (segment (start 153 74.13) (end 153 75.355) (width 0.25) (layer F.Cu) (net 8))
 (segment (start 158.670001 80.140002) (end 159.5 79.310003) (width 0.25) (layer F.Cu) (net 8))
 (segment (start 154.230002 80.140002) (end 158.670001 80.140002) (width 0.25) (layer F.Cu) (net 8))
 (segment (start 154.1 80.01) (end 154.230002 80.140002) (width 0.25) (layer F.Cu) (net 8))
 (segment (start 153 80.01) (end 154.1 80.01) (width 0.25) (layer F.Cu) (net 8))
 (segment (start 159.5 76.770003) (end 160.324999 75.945004) (width 0.25) (layer F.Cu) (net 8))
 (segment (start 159.5 79.310003) (end 159.5 76.770003) (width 0.25) (layer F.Cu) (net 8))
 (segment (start 158.670001 77.600002) (end 159.5 76.770003) (width 0.25) (layer F.Cu) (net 8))
 (segment (start 153 72.905) (end 153 61.83) (width 0.25) (layer F.Cu) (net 8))
 (segment (start 153 74.13) (end 153 72.905) (width 0.25) (layer F.Cu) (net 8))
 (segment (start 153 49.53) (end 153 55.68) (width 0.25) (layer B.Cu) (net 8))
 (segment (start 153 55.68) (end 153 61.83) (width 0.25) (layer F.Cu) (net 8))
 (segment (start 153.594999 61.235001) (end 153 61.83) (width 0.25) (layer F.Cu) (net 8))
 (segment (start 158.13 61.235001) (end 153.594999 61.235001) (width 0.25) (layer F.Cu) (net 8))
 (segment (start 139.849999 80.009999) (end 139 79.16) (width 0.25) (layer F.Cu) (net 2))
 (segment (start 141 81.16) (end 139.849999 80.009999) (width 0.25) (layer F.Cu) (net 2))
 (segment (start 141 87.285001) (end 141 81.16) (width 0.25) (layer F.Cu) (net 2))
 (segment (start 142.89 89.175001) (end 141 87.285001) (width 0.25) (layer F.Cu) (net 2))
 (segment (start 141.764999 89.715002) (end 142.549997 90.5) (width 0.25) (layer B.Cu) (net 1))
 (segment (start 141.764999 87.139997) (end 141.764999 89.715002) (width 0.25) (layer B.Cu) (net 1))
 (segment (start 139 84.374998) (end 141.764999 87.139997) (width 0.25) (layer B.Cu) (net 1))
 (segment (start 139 81.7) (end 139 84.374998) (width 0.25) (layer B.Cu) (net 1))
 (segment (start 156.805001 90.5) (end 158.13 89.175001) (width 0.25) (layer B.Cu) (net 1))
 (segment (start 142.549997 90.5) (end 156.805001 90.5) (width 0.25) (layer B.Cu) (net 1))
 (segment (start 164.200001 41.639999) (end 165 40.84) (width 0.25) (layer B.Cu) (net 27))
 (segment (start 163.874999 41.965001) (end 164.200001 41.639999) (width 0.25) (layer B.Cu) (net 27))
 (segment (start 158.565001 41.965001) (end 163.874999 41.965001) (width 0.25) (layer B.Cu) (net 27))
 (segment (start 157.6 41) (end 158.565001 41.965001) (width 0.25) (layer B.Cu) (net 27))
 (segment (start 156.5 41) (end 157.6 41) (width 0.25) (layer B.Cu) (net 27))
 (segment (start 161.200001 40.040001) (end 162 40.84) (width 0.25) (layer B.Cu) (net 28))
 (segment (start 160.984999 39.824999) (end 161.200001 40.040001) (width 0.25) (layer B.Cu) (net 28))
 (segment (start 155.135001 39.824999) (end 160.984999 39.824999) (width 0.25) (layer B.Cu) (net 28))
 (segment (start 153.96 41) (end 155.135001 39.824999) (width 0.25) (layer B.Cu) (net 28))
 (segment (start 149.780001 42.639999) (end 150.570001 41.849999) (width 0.25) (layer B.Cu) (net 29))
 (segment (start 150.570001 41.849999) (end 151.42 41) (width 0.25) (layer B.Cu) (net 29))
 (segment (start 140.299999 42.639999) (end 149.780001 42.639999) (width 0.25) (layer B.Cu) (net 29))
 (segment (start 139.5 41.84) (end 140.299999 42.639999) (width 0.25) (layer B.Cu) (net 29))
 (segment (start 148.030001 40.150001) (end 148.88 41) (width 0.25) (layer B.Cu) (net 30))
 (segment (start 147.38 39.5) (end 148.030001 40.150001) (width 0.25) (layer B.Cu) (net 30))
 (segment (start 138.84 39.5) (end 147.38 39.5) (width 0.25) (layer B.Cu) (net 30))
 (segment (start 136.5 41.84) (end 138.84 39.5) (width 0.25) (layer B.Cu) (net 30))
 (segment (start 145.490001 41.849999) (end 146.34 41) (width 0.25) (layer F.Cu) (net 31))
 (segment (start 143.885997 42.175001) (end 145.164999 42.175001) (width 0.25) (layer F.Cu) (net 31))
 (segment (start 142.5 43.560998) (end 143.885997 42.175001) (width 0.25) (layer F.Cu) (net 31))
 (segment (start 145.164999 42.175001) (end 145.490001 41.849999) (width 0.25) (layer F.Cu) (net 31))
 (segment (start 142.5 51.34) (end 142.5 43.560998) (width 0.25) (layer F.Cu) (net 31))
 (segment (start 139.5 54.34) (end 142.5 51.34) (width 0.25) (layer F.Cu) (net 31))
 (segment (start 142.950001 41.849999) (end 143.8 41) (width 0.25) (layer F.Cu) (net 32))
 (segment (start 137.625001 47.174999) (end 142.950001 41.849999) (width 0.25) (layer F.Cu) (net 32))
 (segment (start 137.625001 53.214999) (end 137.625001 47.174999) (width 0.25) (layer F.Cu) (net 32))
 (segment (start 136.5 54.34) (end 137.625001 53.214999) (width 0.25) (layer F.Cu) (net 32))
 (segment (start 158.144999 53.63) (end 158.13 53.615001) (width 0.25) (layer B.Cu) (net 3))
 (segment (start 161 53.63) (end 158.144999 53.63) (width 0.25) (layer B.Cu) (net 3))
 (segment (start 139.849999 77.469999) (end 139 76.62) (width 0.25) (layer F.Cu) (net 4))
 (segment (start 141.45001 79.07001) (end 139.849999 77.469999) (width 0.25) (layer F.Cu) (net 4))
 (segment (start 141.45001 85.195011) (end 141.45001 79.07001) (width 0.25) (layer F.Cu) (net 4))
 (segment (start 142.89 86.635001) (end 141.45001 85.195011) (width 0.25) (layer F.Cu) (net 4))
 (segment (start 139 74.5) (end 139 74.08) (width 0.25) (layer B.Cu) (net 6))
 (segment (start 140.175001 75.675001) (end 139 74.5) (width 0.25) (layer B.Cu) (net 6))
 (segment (start 140.175001 81.380002) (end 140.175001 75.675001) (width 0.25) (layer B.Cu) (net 6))
 (segment (start 142.89 84.095001) (end 140.175001 81.380002) (width 0.25) (layer B.Cu) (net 6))
 (segment (start 139.849999 72.389999) (end 139 71.54) (width 0.25) (layer B.Cu) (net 7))
 (segment (start 140.625011 79.290012) (end 140.625011 73.165011) (width 0.25) (layer B.Cu) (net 7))
 (segment (start 140.625011 73.165011) (end 139.849999 72.389999) (width 0.25) (layer B.Cu) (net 7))
 (segment (start 142.89 81.555001) (end 140.625011 79.290012) (width 0.25) (layer B.Cu) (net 7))
 (segment (start 139 67.665001) (end 142.89 63.775001) (width 0.25) (layer B.Cu) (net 21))
 (segment (start 139 69) (end 139 67.665001) (width 0.25) (layer B.Cu) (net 21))
 (segment (start 149.24 86.22) (end 149.24 85.09) (width 0.25) (layer B.Cu) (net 24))
 (segment (start 146.46 89) (end 149.24 86.22) (width 0.25) (layer B.Cu) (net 24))
 (segment (start 144.015001 57.280002) (end 144.015001 83.015001) (width 0.25) (layer F.Cu) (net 24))
 (segment (start 142.89 56.155001) (end 144.015001 57.280002) (width 0.25) (layer F.Cu) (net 24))
 (segment (start 147.165001 83.015001) (end 149.24 85.09) (width 0.25) (layer F.Cu) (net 24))
 (segment (start 144.015001 83.015001) (end 147.165001 83.015001) (width 0.25) (layer F.Cu) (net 24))
 (segment (start 156.99863 86.635001) (end 158.13 86.635001) (width 0.25) (layer F.Cu) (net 25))
 (segment (start 152.12292 86.635001) (end 156.99863 86.635001) (width 0.25) (layer F.Cu) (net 25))
 (segment (start 151.78 86.292081) (end 152.12292 86.635001) (width 0.25) (layer F.Cu) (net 25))
 (segment (start 151.78 85.09) (end 151.78 86.292081) (width 0.25) (layer F.Cu) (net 25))
 (segment (start 150.930001 85.939999) (end 151.78 85.09) (width 0.25) (layer F.Cu) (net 25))
 (segment (start 146.775001 86.265001) (end 150.604999 86.265001) (width 0.25) (layer F.Cu) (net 25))
 (segment (start 150.604999 86.265001) (end 150.930001 85.939999) (width 0.25) (layer F.Cu) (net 25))
 (segment (start 146.7 86.19) (end 146.775001 86.265001) (width 0.25) (layer F.Cu) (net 25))
 (segment (start 146.7 85.09) (end 146.7 86.19) (width 0.25) (layer F.Cu) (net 25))
 (segment (start 154.32 88.78) (end 154.54 89) (width 0.25) (layer B.Cu) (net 26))
 (segment (start 154.32 85.09) (end 154.32 88.78) (width 0.25) (layer B.Cu) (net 26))
 (segment (start 152.73 83.5) (end 154.32 85.09) (width 0.25) (layer F.Cu) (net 26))
 (segment (start 148.28641 83.5) (end 152.73 83.5) (width 0.25) (layer F.Cu) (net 26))
 (segment (start 144.5 54.175001) (end 144.5 82.5) (width 0.25) (layer F.Cu) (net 26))
 (segment (start 147.28641 82.5) (end 148.28641 83.5) (width 0.25) (layer F.Cu) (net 26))
 (segment (start 144.5 82.5) (end 147.28641 82.5) (width 0.25) (layer F.Cu) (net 26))
 (segment (start 143.94 53.615001) (end 144.5 54.175001) (width 0.25) (layer F.Cu) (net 26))
 (segment (start 142.89 53.615001) (end 143.94 53.615001) (width 0.25) (layer F.Cu) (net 26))
 (segment (start 156.5 44) (end 143.8 44) (width 0.25) (layer B.Cu) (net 5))
 (segment (start 148 44.88) (end 148 49.53) (width 0.25) (layer F.Cu) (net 5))
 (segment (start 148.88 44) (end 148 44.88) (width 0.25) (layer F.Cu) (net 5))
 (segment (start 148 49.53) (end 148 80.01) (width 0.25) (layer F.Cu) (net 5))
 (segment (start 158.144999 56.17) (end 158.13 56.155001) (width 0.25) (layer B.Cu) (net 5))
 (segment (start 161 56.17) (end 158.144999 56.17) (width 0.25) (layer B.Cu) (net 5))
 (segment (start 156.354989 54.37999) (end 157.330001 55.355002) (width 0.25) (layer F.Cu) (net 5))
 (segment (start 149.17501 54.37999) (end 156.354989 54.37999) (width 0.25) (layer F.Cu) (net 5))
 (segment (start 157.330001 55.355002) (end 158.13 56.155001) (width 0.25) (layer F.Cu) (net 5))
 (segment (start 148 55.555) (end 149.17501 54.37999) (width 0.25) (layer F.Cu) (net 5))
 (segment (start 148 55.68) (end 148 55.555) (width 0.25) (layer F.Cu) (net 5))
 (segment (start 153.239998 87.760002) (end 152 89) (width 0.25) (layer F.Cu) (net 5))
 (segment (start 159.255001 87.175002) (end 158.670001 87.760002) (width 0.25) (layer F.Cu) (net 5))
 (segment (start 159.255001 86.095) (end 159.255001 87.175002) (width 0.25) (layer F.Cu) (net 5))
 (segment (start 158.670001 85.51) (end 159.255001 86.095) (width 0.25) (layer F.Cu) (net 5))
 (segment (start 152.974013 82.005011) (end 156.479002 85.51) (width 0.25) (layer F.Cu) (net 5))
 (segment (start 149.995011 82.005011) (end 152.974013 82.005011) (width 0.25) (layer F.Cu) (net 5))
 (segment (start 158.670001 87.760002) (end 153.239998 87.760002) (width 0.25) (layer F.Cu) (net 5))
 (segment (start 156.479002 85.51) (end 158.670001 85.51) (width 0.25) (layer F.Cu) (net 5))
 (segment (start 148 80.01) (end 149.995011 82.005011) (width 0.25) (layer F.Cu) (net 5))
 (segment (start 149 89) (end 152 89) (width 0.25) (layer B.Cu) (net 5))
 (segment (start 151.470002 77.600002) (end 148 74.13) (width 0.25) (layer B.Cu) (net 5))
 (segment (start 159.439998 77.600002) (end 151.470002 77.600002) (width 0.25) (layer B.Cu) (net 5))
 (segment (start 161.5 75.54) (end 159.439998 77.600002) (width 0.25) (layer B.Cu) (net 5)))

